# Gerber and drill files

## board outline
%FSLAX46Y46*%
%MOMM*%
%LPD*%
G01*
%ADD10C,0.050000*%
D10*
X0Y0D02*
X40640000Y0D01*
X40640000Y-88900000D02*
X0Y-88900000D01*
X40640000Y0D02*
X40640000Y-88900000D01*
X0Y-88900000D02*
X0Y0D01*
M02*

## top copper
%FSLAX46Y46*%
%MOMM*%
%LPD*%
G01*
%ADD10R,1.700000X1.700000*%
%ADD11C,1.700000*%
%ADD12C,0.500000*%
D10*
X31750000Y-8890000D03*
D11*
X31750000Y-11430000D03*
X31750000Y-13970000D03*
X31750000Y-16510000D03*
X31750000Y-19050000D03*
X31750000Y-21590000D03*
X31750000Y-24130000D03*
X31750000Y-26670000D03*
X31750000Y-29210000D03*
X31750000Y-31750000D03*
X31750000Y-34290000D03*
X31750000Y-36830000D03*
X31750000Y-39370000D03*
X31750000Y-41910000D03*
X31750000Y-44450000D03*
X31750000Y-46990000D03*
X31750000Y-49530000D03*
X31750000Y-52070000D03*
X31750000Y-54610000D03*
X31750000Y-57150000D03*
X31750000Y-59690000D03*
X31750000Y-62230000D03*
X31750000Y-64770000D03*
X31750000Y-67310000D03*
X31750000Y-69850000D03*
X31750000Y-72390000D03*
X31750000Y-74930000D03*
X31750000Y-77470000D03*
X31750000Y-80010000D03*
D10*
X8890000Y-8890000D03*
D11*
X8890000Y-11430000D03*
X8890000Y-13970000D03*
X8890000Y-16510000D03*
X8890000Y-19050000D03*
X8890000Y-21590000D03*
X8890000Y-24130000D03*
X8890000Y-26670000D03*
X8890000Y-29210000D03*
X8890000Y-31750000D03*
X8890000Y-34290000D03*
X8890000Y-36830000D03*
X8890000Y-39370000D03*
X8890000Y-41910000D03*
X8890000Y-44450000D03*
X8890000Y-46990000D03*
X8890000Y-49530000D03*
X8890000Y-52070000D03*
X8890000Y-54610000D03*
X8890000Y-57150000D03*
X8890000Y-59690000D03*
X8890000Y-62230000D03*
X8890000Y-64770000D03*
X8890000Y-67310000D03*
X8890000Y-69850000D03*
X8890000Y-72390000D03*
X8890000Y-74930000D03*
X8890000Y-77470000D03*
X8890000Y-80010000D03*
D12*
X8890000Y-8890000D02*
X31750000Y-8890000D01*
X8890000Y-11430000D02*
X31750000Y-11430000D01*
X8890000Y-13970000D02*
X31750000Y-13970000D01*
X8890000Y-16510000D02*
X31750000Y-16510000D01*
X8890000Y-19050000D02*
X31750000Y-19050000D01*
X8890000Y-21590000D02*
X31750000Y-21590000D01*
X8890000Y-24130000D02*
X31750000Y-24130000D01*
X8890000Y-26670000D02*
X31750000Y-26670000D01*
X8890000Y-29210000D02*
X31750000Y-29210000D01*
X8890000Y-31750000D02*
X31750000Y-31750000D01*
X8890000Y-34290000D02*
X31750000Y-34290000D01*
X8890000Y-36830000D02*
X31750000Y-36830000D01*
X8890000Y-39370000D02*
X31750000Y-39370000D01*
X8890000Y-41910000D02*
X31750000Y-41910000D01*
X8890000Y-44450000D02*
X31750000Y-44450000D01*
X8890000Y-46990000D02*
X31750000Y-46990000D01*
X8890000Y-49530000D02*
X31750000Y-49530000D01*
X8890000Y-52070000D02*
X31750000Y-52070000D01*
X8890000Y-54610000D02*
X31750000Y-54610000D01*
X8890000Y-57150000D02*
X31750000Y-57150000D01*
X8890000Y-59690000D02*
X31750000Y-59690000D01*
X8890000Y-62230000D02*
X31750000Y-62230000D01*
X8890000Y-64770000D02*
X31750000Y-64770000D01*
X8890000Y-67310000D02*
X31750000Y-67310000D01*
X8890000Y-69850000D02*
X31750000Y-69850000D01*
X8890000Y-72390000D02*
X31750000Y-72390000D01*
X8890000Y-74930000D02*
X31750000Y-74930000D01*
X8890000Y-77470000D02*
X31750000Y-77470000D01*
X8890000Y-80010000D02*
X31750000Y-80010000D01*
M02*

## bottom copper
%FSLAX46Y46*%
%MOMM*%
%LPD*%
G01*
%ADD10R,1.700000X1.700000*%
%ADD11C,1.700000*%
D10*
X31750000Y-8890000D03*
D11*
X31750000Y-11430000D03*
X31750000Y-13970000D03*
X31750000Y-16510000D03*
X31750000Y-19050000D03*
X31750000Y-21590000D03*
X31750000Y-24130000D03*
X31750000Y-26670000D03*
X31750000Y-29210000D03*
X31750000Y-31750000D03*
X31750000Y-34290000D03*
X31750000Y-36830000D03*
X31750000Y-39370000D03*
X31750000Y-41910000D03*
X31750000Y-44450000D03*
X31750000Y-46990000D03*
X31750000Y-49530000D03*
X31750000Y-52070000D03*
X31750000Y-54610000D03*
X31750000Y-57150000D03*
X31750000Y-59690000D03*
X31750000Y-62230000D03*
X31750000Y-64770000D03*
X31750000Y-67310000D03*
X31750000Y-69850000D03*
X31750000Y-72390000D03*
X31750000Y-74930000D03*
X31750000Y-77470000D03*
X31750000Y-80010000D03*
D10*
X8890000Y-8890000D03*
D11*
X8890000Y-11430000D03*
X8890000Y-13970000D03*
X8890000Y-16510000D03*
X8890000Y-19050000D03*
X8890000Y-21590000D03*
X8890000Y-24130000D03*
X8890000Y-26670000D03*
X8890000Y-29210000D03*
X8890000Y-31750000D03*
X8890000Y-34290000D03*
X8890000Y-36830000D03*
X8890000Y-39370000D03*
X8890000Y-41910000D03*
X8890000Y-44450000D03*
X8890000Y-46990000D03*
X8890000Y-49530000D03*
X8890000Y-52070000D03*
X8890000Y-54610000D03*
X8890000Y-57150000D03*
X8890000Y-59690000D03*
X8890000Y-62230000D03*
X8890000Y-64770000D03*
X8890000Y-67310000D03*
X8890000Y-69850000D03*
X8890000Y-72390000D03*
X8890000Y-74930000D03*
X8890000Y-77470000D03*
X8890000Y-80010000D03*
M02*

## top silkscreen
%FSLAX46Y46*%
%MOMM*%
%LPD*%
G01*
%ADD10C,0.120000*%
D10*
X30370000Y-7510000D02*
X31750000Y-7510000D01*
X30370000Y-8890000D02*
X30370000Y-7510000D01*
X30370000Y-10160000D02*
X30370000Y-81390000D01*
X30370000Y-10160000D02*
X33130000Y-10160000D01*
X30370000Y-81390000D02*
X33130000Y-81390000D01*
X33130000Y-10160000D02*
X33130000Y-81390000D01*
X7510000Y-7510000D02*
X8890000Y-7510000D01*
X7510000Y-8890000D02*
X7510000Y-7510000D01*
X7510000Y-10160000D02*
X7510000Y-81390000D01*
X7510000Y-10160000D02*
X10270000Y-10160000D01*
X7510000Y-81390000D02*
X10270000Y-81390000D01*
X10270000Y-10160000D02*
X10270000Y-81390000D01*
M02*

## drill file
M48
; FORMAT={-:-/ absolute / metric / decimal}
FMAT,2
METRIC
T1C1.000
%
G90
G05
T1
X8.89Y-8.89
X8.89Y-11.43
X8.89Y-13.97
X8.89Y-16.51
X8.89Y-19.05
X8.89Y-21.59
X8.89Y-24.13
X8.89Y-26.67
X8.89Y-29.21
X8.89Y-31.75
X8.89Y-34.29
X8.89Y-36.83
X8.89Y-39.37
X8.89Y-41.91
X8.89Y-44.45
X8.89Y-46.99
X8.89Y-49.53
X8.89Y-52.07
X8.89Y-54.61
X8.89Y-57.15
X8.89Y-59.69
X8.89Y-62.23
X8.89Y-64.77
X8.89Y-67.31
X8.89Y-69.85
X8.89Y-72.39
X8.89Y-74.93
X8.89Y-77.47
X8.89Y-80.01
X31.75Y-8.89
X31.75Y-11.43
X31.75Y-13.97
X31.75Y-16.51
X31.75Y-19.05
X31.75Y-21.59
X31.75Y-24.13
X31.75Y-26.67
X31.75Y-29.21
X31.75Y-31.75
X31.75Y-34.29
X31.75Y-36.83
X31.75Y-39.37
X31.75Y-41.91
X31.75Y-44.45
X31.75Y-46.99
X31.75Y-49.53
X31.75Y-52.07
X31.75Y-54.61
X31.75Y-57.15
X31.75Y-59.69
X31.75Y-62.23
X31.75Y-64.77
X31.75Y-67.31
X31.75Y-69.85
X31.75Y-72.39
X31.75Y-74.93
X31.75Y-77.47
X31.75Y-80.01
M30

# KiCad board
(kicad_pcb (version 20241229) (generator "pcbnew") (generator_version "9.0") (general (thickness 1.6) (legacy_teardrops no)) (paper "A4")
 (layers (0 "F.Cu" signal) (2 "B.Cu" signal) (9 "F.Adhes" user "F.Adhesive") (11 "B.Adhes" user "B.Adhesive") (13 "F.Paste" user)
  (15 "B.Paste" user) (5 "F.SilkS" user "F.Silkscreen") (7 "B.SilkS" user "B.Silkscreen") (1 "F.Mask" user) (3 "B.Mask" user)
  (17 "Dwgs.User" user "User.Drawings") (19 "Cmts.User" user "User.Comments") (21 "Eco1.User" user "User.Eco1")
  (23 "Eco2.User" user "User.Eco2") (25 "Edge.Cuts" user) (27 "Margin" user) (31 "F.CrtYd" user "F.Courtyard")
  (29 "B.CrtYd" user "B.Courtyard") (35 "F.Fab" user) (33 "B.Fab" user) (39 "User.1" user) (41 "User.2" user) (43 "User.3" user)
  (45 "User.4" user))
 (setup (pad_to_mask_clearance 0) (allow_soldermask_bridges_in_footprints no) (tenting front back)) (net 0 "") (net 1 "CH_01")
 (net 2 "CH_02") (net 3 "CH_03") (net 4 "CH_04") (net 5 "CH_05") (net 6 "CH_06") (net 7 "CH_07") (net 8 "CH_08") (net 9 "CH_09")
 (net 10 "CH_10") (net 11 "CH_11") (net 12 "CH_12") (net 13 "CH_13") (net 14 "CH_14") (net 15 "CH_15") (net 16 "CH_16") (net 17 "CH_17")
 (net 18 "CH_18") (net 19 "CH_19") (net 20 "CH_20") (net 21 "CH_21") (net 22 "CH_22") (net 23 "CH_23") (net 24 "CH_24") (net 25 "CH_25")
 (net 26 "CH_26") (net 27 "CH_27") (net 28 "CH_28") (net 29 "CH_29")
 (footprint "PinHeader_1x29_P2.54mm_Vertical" (layer "F.Cu") (at 31.75 8.89)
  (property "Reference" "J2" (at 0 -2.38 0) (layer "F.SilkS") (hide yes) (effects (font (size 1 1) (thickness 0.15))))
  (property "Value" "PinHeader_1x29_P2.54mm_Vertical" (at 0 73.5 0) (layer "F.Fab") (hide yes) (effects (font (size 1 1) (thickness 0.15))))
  (fp_line (start -1.38 -1.38) (end 0 -1.38) (stroke (width 0.12) (type solid)) (layer "F.SilkS"))
  (fp_line (start -1.38 0) (end -1.38 -1.38) (stroke (width 0.12) (type solid)) (layer "F.SilkS"))
  (fp_line (start -1.38 1.27) (end -1.38 72.5) (stroke (width 0.12) (type solid)) (layer "F.SilkS"))
  (fp_line (start -1.38 1.27) (end 1.38 1.27) (stroke (width 0.12) (type solid)) (layer "F.SilkS"))
  (fp_line (start -1.38 72.5) (end 1.38 72.5) (stroke (width 0.12) (type solid)) (layer "F.SilkS"))
  (fp_line (start 1.38 1.27) (end 1.38 72.5) (stroke (width 0.12) (type solid)) (layer "F.SilkS"))
  (pad "1" thru_hole rect (at 0 0) (size 1.7 1.7) (drill 1) (layers "*.Cu" "*.Mask") (remove_unused_layers no) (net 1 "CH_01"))
  (pad "2" thru_hole circle (at 0 2.54) (size 1.7 1.7) (drill 1) (layers "*.Cu" "*.Mask") (remove_unused_layers no) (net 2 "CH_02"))
  (pad "3" thru_hole circle (at 0 5.08) (size 1.7 1.7) (drill 1) (layers "*.Cu" "*.Mask") (remove_unused_layers no) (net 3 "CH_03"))
  (pad "4" thru_hole circle (at 0 7.62) (size 1.7 1.7) (drill 1) (layers "*.Cu" "*.Mask") (remove_unused_layers no) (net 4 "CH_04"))
  (pad "5" thru_hole circle (at 0 10.16) (size 1.7 1.7) (drill 1) (layers "*.Cu" "*.Mask") (remove_unused_layers no) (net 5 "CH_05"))
  (pad "6" thru_hole circle (at 0 12.7) (size 1.7 1.7) (drill 1) (layers "*.Cu" "*.Mask") (remove_unused_layers no) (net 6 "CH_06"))
  (pad "7" thru_hole circle (at 0 15.24) (size 1.7 1.7) (drill 1) (layers "*.Cu" "*.Mask") (remove_unused_layers no) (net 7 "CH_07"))
  (pad "8" thru_hole circle (at 0 17.78) (size 1.7 1.7) (drill 1) (layers "*.Cu" "*.Mask") (remove_unused_layers no) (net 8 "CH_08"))
  (pad "9" thru_hole circle (at 0 20.32) (size 1.7 1.7) (drill 1) (layers "*.Cu" "*.Mask") (remove_unused_layers no) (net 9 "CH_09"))
  (pad "10" thru_hole circle (at 0 22.86) (size 1.7 1.7) (drill 1) (layers "*.Cu" "*.Mask") (remove_unused_layers no) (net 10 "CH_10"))
  (pad "11" thru_hole circle (at 0 25.4) (size 1.7 1.7) (drill 1) (layers "*.Cu" "*.Mask") (remove_unused_layers no) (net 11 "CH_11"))
  (pad "12" thru_hole circle (at 0 27.94) (size 1.7 1.7) (drill 1) (layers "*.Cu" "*.Mask") (remove_unused_layers no) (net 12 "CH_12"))
  (pad "13" thru_hole circle (at 0 30.48) (size 1.7 1.7) (drill 1) (layers "*.Cu" "*.Mask") (remove_unused_layers no) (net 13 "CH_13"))
  (pad "14" thru_hole circle (at 0 33.02) (size 1.7 1.7) (drill 1) (layers "*.Cu" "*.Mask") (remove_unused_layers no) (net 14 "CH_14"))
  (pad "15" thru_hole circle (at 0 35.56) (size 1.7 1.7) (drill 1) (layers "*.Cu" "*.Mask") (remove_unused_layers no) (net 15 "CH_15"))
  (pad "16" thru_hole circle (at 0 38.1) (size 1.7 1.7) (drill 1) (layers "*.Cu" "*.Mask") (remove_unused_layers no) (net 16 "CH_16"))
  (pad "17" thru_hole circle (at 0 40.64) (size 1.7 1.7) (drill 1) (layers "*.Cu" "*.Mask") (remove_unused_layers no) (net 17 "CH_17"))
  (pad "18" thru_hole circle (at 0 43.18) (size 1.7 1.7) (drill 1) (layers "*.Cu" "*.Mask") (remove_unused_layers no) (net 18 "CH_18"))
  (pad "19" thru_hole circle (at 0 45.72) (size 1.7 1.7) (drill 1) (layers "*.Cu" "*.Mask") (remove_unused_layers no) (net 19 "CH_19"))
  (pad "20" thru_hole circle (at 0 48.26) (size 1.7 1.7) (drill 1) (layers "*.Cu" "*.Mask") (remove_unused_layers no) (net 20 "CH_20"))
  (pad "21" thru_hole circle (at 0 50.8) (size 1.7 1.7) (drill 1) (layers "*.Cu" "*.Mask") (remove_unused_layers no) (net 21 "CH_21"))
  (pad "22" thru_hole circle (at 0 53.34) (size 1.7 1.7) (drill 1) (layers "*.Cu" "*.Mask") (remove_unused_layers no) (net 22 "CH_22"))
  (pad "23" thru_hole circle (at 0 55.88) (size 1.7 1.7) (drill 1) (layers "*.Cu" "*.Mask") (remove_unused_layers no) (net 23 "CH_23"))
  (pad "24" thru_hole circle (at 0 58.42) (size 1.7 1.7) (drill 1) (layers "*.Cu" "*.Mask") (remove_unused_layers no) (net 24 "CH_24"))
  (pad "25" thru_hole circle (at 0 60.96) (size 1.7 1.7) (drill 1) (layers "*.Cu" "*.Mask") (remove_unused_layers no) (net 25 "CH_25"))
  (pad "26" thru_hole circle (at 0 63.5) (size 1.7 1.7) (drill 1) (layers "*.Cu" "*.Mask") (remove_unused_layers no) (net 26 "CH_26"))
  (pad "27" thru_hole circle (at 0 66.04) (size 1.7 1.7) (drill 1) (layers "*.Cu" "*.Mask") (remove_unused_layers no) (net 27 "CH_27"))
  (pad "28" thru_hole circle (at 0 68.58) (size 1.7 1.7) (drill 1) (layers "*.Cu" "*.Mask") (remove_unused_layers no) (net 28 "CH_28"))
  (pad "29" thru_hole circle (at 0 71.12) (size 1.7 1.7) (drill 1) (layers "*.Cu" "*.Mask") (remove_unused_layers no) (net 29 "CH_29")))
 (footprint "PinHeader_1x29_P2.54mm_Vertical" (layer "F.Cu") (at 8.89 8.89)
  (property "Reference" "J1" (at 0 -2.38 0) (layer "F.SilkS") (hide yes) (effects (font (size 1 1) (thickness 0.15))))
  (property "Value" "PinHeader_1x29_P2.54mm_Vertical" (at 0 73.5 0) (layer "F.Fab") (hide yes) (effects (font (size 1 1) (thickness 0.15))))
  (fp_line (start -1.38 -1.38) (end 0 -1.38) (stroke (width 0.12) (type solid)) (layer "F.SilkS"))
  (fp_line (start -1.38 0) (end -1.38 -1.38) (stroke (width 0.12) (type solid)) (layer "F.SilkS"))
  (fp_line (start -1.38 1.27) (end -1.38 72.5) (stroke (width 0.12) (type solid)) (layer "F.SilkS"))
  (fp_line (start -1.38 1.27) (end 1.38 1.27) (stroke (width 0.12) (type solid)) (layer "F.SilkS"))
  (fp_line (start -1.38 72.5) (end 1.38 72.5) (stroke (width 0.12) (type solid)) (layer "F.SilkS"))
  (fp_line (start 1.38 1.27) (end 1.38 72.5) (stroke (width 0.12) (type solid)) (layer "F.SilkS"))
  (pad "1" thru_hole rect (at 0 0) (size 1.7 1.7) (drill 1) (layers "*.Cu" "*.Mask") (remove_unused_layers no) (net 1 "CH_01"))
  (pad "2" thru_hole circle (at 0 2.54) (size 1.7 1.7) (drill 1) (layers "*.Cu" "*.Mask") (remove_unused_layers no) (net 2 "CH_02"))
  (pad "3" thru_hole circle (at 0 5.08) (size 1.7 1.7) (drill 1) (layers "*.Cu" "*.Mask") (remove_unused_layers no) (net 3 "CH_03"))
  (pad "4" thru_hole circle (at 0 7.62) (size 1.7 1.7) (drill 1) (layers "*.Cu" "*.Mask") (remove_unused_layers no) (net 4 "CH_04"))
  (pad "5" thru_hole circle (at 0 10.16) (size 1.7 1.7) (drill 1) (layers "*.Cu" "*.Mask") (remove_unused_layers no) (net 5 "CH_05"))
  (pad "6" thru_hole circle (at 0 12.7) (size 1.7 1.7) (drill 1) (layers "*.Cu" "*.Mask") (remove_unused_layers no) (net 6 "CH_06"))
  (pad "7" thru_hole circle (at 0 15.24) (size 1.7 1.7) (drill 1) (layers "*.Cu" "*.Mask") (remove_unused_layers no) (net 7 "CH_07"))
  (pad "8" thru_hole circle (at 0 17.78) (size 1.7 1.7) (drill 1) (layers "*.Cu" "*.Mask") (remove_unused_layers no) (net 8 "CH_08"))
  (pad "9" thru_hole circle (at 0 20.32) (size 1.7 1.7) (drill 1) (layers "*.Cu" "*.Mask") (remove_unused_layers no) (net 9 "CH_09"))
  (pad "10" thru_hole circle (at 0 22.86) (size 1.7 1.7) (drill 1) (layers "*.Cu" "*.Mask") (remove_unused_layers no) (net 10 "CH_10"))
  (pad "11" thru_hole circle (at 0 25.4) (size 1.7 1.7) (drill 1) (layers "*.Cu" "*.Mask") (remove_unused_layers no) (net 11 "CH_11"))
  (pad "12" thru_hole circle (at 0 27.94) (size 1.7 1.7) (drill 1) (layers "*.Cu" "*.Mask") (remove_unused_layers no) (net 12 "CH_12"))
  (pad "13" thru_hole circle (at 0 30.48) (size 1.7 1.7) (drill 1) (layers "*.Cu" "*.Mask") (remove_unused_layers no) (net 13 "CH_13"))
  (pad "14" thru_hole circle (at 0 33.02) (size 1.7 1.7) (drill 1) (layers "*.Cu" "*.Mask") (remove_unused_layers no) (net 14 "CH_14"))
  (pad "15" thru_hole circle (at 0 35.56) (size 1.7 1.7) (drill 1) (layers "*.Cu" "*.Mask") (remove_unused_layers no) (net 15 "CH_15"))
  (pad "16" thru_hole circle (at 0 38.1) (size 1.7 1.7) (drill 1) (layers "*.Cu" "*.Mask") (remove_unused_layers no) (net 16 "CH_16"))
  (pad "17" thru_hole circle (at 0 40.64) (size 1.7 1.7) (drill 1) (layers "*.Cu" "*.Mask") (remove_unused_layers no) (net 17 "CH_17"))
  (pad "18" thru_hole circle (at 0 43.18) (size 1.7 1.7) (drill 1) (layers "*.Cu" "*.Mask") (remove_unused_layers no) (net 18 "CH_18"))
  (pad "19" thru_hole circle (at 0 45.72) (size 1.7 1.7) (drill 1) (layers "*.Cu" "*.Mask") (remove_unused_layers no) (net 19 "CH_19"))
  (pad "20" thru_hole circle (at 0 48.26) (size 1.7 1.7) (drill 1) (layers "*.Cu" "*.Mask") (remove_unused_layers no) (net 20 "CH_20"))
  (pad "21" thru_hole circle (at 0 50.8) (size 1.7 1.7) (drill 1) (layers "*.Cu" "*.Mask") (remove_unused_layers no) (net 21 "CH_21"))
  (pad "22" thru_hole circle (at 0 53.34) (size 1.7 1.7) (drill 1) (layers "*.Cu" "*.Mask") (remove_unused_layers no) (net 22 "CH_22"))
  (pad "23" thru_hole circle (at 0 55.88) (size 1.7 1.7) (drill 1) (layers "*.Cu" "*.Mask") (remove_unused_layers no) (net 23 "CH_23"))
  (pad "24" thru_hole circle (at 0 58.42) (size 1.7 1.7) (drill 1) (layers "*.Cu" "*.Mask") (remove_unused_layers no) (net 24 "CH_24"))
  (pad "25" thru_hole circle (at 0 60.96) (size 1.7 1.7) (drill 1) (layers "*.Cu" "*.Mask") (remove_unused_layers no) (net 25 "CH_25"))
  (pad "26" thru_hole circle (at 0 63.5) (size 1.7 1.7) (drill 1) (layers "*.Cu" "*.Mask") (remove_unused_layers no) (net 26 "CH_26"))
  (pad "27" thru_hole circle (at 0 66.04) (size 1.7 1.7) (drill 1) (layers "*.Cu" "*.Mask") (remove_unused_layers no) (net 27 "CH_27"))
  (pad "28" thru_hole circle (at 0 68.58) (size 1.7 1.7) (drill 1) (layers "*.Cu" "*.Mask") (remove_unused_layers no) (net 28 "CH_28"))
  (pad "29" thru_hole circle (at 0 71.12) (size 1.7 1.7) (drill 1) (layers "*.Cu" "*.Mask") (remove_unused_layers no) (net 29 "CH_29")))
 (gr_line (start 0 0) (end 40.64 0) (stroke (width 0.05) (type default)) (layer "Edge.Cuts"))
 (gr_line (start 40.64 88.9) (end 0 88.9) (stroke (width 0.05) (type default)) (layer "Edge.Cuts"))
 (gr_line (start 40.64 0) (end 40.64 88.9) (stroke (width 0.05) (type default)) (layer "Edge.Cuts"))
 (gr_line (start 0 88.9) (end 0 0) (stroke (width 0.05) (type default)) (layer "Edge.Cuts"))
 (segment (start 8.89 8.89) (end 31.75 8.89) (width 0.5) (layer "F.Cu") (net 1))
 (segment (start 8.89 11.43) (end 31.75 11.43) (width 0.5) (layer "F.Cu") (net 2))
 (segment (start 8.89 13.97) (end 31.75 13.97) (width 0.5) (layer "F.Cu") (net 3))
 (segment (start 8.89 16.51) (end 31.75 16.51) (width 0.5) (layer "F.Cu") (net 4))
 (segment (start 8.89 19.05) (end 31.75 19.05) (width 0.5) (layer "F.Cu") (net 5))
 (segment (start 8.89 21.59) (end 31.75 21.59) (width 0.5) (layer "F.Cu") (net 6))
 (segment (start 8.89 24.13) (end 31.75 24.13) (width 0.5) (layer "F.Cu") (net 7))
 (segment (start 8.89 26.67) (end 31.75 26.67) (width 0.5) (layer "F.Cu") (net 8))
 (segment (start 8.89 29.21) (end 31.75 29.21) (width 0.5) (layer "F.Cu") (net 9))
 (segment (start 8.89 31.75) (end 31.75 31.75) (width 0.5) (layer "F.Cu") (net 10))
 (segment (start 8.89 34.29) (end 31.75 34.29) (width 0.5) (layer "F.Cu") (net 11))
 (segment (start 8.89 36.83) (end 31.75 36.83) (width 0.5) (layer "F.Cu") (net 12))
 (segment (start 8.89 39.37) (end 31.75 39.37) (width 0.5) (layer "F.Cu") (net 13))
 (segment (start 8.89 41.91) (end 31.75 41.91) (width 0.5) (layer "F.Cu") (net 14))
 (segment (start 8.89 44.45) (end 31.75 44.45) (width 0.5) (layer "F.Cu") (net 15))
 (segment (start 8.89 46.99) (end 31.75 46.99) (width 0.5) (layer "F.Cu") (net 16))
 (segment (start 8.89 49.53) (end 31.75 49.53) (width 0.5) (layer "F.Cu") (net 17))
 (segment (start 8.89 52.07) (end 31.75 52.07) (width 0.5) (layer "F.Cu") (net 18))
 (segment (start 8.89 54.61) (end 31.75 54.61) (width 0.5) (layer "F.Cu") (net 19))
 (segment (start 8.89 57.15) (end 31.75 57.15) (width 0.5) (layer "F.Cu") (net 20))
 (segment (start 8.89 59.69) (end 31.75 59.69) (width 0.5) (layer "F.Cu") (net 21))
 (segment (start 8.89 62.23) (end 31.75 62.23) (width 0.5) (layer "F.Cu") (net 22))
 (segment (start 8.89 64.77) (end 31.75 64.77) (width 0.5) (layer "F.Cu") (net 23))
 (segment (start 8.89 67.31) (end 31.75 67.31) (width 0.5) (layer "F.Cu") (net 24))
 (segment (start 8.89 69.85) (end 31.75 69.85) (width 0.5) (layer "F.Cu") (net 25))
 (segment (start 8.89 72.39) (end 31.75 72.39) (width 0.5) (layer "F.Cu") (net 26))
 (segment (start 8.89 74.93) (end 31.75 74.93) (width 0.5) (layer "F.Cu") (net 27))
 (segment (start 8.89 77.47) (end 31.75 77.47) (width 0.5) (layer "F.Cu") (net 28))
 (segment (start 8.89 80.01) (end 31.75 80.01) (width 0.5) (layer "F.Cu") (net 29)))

